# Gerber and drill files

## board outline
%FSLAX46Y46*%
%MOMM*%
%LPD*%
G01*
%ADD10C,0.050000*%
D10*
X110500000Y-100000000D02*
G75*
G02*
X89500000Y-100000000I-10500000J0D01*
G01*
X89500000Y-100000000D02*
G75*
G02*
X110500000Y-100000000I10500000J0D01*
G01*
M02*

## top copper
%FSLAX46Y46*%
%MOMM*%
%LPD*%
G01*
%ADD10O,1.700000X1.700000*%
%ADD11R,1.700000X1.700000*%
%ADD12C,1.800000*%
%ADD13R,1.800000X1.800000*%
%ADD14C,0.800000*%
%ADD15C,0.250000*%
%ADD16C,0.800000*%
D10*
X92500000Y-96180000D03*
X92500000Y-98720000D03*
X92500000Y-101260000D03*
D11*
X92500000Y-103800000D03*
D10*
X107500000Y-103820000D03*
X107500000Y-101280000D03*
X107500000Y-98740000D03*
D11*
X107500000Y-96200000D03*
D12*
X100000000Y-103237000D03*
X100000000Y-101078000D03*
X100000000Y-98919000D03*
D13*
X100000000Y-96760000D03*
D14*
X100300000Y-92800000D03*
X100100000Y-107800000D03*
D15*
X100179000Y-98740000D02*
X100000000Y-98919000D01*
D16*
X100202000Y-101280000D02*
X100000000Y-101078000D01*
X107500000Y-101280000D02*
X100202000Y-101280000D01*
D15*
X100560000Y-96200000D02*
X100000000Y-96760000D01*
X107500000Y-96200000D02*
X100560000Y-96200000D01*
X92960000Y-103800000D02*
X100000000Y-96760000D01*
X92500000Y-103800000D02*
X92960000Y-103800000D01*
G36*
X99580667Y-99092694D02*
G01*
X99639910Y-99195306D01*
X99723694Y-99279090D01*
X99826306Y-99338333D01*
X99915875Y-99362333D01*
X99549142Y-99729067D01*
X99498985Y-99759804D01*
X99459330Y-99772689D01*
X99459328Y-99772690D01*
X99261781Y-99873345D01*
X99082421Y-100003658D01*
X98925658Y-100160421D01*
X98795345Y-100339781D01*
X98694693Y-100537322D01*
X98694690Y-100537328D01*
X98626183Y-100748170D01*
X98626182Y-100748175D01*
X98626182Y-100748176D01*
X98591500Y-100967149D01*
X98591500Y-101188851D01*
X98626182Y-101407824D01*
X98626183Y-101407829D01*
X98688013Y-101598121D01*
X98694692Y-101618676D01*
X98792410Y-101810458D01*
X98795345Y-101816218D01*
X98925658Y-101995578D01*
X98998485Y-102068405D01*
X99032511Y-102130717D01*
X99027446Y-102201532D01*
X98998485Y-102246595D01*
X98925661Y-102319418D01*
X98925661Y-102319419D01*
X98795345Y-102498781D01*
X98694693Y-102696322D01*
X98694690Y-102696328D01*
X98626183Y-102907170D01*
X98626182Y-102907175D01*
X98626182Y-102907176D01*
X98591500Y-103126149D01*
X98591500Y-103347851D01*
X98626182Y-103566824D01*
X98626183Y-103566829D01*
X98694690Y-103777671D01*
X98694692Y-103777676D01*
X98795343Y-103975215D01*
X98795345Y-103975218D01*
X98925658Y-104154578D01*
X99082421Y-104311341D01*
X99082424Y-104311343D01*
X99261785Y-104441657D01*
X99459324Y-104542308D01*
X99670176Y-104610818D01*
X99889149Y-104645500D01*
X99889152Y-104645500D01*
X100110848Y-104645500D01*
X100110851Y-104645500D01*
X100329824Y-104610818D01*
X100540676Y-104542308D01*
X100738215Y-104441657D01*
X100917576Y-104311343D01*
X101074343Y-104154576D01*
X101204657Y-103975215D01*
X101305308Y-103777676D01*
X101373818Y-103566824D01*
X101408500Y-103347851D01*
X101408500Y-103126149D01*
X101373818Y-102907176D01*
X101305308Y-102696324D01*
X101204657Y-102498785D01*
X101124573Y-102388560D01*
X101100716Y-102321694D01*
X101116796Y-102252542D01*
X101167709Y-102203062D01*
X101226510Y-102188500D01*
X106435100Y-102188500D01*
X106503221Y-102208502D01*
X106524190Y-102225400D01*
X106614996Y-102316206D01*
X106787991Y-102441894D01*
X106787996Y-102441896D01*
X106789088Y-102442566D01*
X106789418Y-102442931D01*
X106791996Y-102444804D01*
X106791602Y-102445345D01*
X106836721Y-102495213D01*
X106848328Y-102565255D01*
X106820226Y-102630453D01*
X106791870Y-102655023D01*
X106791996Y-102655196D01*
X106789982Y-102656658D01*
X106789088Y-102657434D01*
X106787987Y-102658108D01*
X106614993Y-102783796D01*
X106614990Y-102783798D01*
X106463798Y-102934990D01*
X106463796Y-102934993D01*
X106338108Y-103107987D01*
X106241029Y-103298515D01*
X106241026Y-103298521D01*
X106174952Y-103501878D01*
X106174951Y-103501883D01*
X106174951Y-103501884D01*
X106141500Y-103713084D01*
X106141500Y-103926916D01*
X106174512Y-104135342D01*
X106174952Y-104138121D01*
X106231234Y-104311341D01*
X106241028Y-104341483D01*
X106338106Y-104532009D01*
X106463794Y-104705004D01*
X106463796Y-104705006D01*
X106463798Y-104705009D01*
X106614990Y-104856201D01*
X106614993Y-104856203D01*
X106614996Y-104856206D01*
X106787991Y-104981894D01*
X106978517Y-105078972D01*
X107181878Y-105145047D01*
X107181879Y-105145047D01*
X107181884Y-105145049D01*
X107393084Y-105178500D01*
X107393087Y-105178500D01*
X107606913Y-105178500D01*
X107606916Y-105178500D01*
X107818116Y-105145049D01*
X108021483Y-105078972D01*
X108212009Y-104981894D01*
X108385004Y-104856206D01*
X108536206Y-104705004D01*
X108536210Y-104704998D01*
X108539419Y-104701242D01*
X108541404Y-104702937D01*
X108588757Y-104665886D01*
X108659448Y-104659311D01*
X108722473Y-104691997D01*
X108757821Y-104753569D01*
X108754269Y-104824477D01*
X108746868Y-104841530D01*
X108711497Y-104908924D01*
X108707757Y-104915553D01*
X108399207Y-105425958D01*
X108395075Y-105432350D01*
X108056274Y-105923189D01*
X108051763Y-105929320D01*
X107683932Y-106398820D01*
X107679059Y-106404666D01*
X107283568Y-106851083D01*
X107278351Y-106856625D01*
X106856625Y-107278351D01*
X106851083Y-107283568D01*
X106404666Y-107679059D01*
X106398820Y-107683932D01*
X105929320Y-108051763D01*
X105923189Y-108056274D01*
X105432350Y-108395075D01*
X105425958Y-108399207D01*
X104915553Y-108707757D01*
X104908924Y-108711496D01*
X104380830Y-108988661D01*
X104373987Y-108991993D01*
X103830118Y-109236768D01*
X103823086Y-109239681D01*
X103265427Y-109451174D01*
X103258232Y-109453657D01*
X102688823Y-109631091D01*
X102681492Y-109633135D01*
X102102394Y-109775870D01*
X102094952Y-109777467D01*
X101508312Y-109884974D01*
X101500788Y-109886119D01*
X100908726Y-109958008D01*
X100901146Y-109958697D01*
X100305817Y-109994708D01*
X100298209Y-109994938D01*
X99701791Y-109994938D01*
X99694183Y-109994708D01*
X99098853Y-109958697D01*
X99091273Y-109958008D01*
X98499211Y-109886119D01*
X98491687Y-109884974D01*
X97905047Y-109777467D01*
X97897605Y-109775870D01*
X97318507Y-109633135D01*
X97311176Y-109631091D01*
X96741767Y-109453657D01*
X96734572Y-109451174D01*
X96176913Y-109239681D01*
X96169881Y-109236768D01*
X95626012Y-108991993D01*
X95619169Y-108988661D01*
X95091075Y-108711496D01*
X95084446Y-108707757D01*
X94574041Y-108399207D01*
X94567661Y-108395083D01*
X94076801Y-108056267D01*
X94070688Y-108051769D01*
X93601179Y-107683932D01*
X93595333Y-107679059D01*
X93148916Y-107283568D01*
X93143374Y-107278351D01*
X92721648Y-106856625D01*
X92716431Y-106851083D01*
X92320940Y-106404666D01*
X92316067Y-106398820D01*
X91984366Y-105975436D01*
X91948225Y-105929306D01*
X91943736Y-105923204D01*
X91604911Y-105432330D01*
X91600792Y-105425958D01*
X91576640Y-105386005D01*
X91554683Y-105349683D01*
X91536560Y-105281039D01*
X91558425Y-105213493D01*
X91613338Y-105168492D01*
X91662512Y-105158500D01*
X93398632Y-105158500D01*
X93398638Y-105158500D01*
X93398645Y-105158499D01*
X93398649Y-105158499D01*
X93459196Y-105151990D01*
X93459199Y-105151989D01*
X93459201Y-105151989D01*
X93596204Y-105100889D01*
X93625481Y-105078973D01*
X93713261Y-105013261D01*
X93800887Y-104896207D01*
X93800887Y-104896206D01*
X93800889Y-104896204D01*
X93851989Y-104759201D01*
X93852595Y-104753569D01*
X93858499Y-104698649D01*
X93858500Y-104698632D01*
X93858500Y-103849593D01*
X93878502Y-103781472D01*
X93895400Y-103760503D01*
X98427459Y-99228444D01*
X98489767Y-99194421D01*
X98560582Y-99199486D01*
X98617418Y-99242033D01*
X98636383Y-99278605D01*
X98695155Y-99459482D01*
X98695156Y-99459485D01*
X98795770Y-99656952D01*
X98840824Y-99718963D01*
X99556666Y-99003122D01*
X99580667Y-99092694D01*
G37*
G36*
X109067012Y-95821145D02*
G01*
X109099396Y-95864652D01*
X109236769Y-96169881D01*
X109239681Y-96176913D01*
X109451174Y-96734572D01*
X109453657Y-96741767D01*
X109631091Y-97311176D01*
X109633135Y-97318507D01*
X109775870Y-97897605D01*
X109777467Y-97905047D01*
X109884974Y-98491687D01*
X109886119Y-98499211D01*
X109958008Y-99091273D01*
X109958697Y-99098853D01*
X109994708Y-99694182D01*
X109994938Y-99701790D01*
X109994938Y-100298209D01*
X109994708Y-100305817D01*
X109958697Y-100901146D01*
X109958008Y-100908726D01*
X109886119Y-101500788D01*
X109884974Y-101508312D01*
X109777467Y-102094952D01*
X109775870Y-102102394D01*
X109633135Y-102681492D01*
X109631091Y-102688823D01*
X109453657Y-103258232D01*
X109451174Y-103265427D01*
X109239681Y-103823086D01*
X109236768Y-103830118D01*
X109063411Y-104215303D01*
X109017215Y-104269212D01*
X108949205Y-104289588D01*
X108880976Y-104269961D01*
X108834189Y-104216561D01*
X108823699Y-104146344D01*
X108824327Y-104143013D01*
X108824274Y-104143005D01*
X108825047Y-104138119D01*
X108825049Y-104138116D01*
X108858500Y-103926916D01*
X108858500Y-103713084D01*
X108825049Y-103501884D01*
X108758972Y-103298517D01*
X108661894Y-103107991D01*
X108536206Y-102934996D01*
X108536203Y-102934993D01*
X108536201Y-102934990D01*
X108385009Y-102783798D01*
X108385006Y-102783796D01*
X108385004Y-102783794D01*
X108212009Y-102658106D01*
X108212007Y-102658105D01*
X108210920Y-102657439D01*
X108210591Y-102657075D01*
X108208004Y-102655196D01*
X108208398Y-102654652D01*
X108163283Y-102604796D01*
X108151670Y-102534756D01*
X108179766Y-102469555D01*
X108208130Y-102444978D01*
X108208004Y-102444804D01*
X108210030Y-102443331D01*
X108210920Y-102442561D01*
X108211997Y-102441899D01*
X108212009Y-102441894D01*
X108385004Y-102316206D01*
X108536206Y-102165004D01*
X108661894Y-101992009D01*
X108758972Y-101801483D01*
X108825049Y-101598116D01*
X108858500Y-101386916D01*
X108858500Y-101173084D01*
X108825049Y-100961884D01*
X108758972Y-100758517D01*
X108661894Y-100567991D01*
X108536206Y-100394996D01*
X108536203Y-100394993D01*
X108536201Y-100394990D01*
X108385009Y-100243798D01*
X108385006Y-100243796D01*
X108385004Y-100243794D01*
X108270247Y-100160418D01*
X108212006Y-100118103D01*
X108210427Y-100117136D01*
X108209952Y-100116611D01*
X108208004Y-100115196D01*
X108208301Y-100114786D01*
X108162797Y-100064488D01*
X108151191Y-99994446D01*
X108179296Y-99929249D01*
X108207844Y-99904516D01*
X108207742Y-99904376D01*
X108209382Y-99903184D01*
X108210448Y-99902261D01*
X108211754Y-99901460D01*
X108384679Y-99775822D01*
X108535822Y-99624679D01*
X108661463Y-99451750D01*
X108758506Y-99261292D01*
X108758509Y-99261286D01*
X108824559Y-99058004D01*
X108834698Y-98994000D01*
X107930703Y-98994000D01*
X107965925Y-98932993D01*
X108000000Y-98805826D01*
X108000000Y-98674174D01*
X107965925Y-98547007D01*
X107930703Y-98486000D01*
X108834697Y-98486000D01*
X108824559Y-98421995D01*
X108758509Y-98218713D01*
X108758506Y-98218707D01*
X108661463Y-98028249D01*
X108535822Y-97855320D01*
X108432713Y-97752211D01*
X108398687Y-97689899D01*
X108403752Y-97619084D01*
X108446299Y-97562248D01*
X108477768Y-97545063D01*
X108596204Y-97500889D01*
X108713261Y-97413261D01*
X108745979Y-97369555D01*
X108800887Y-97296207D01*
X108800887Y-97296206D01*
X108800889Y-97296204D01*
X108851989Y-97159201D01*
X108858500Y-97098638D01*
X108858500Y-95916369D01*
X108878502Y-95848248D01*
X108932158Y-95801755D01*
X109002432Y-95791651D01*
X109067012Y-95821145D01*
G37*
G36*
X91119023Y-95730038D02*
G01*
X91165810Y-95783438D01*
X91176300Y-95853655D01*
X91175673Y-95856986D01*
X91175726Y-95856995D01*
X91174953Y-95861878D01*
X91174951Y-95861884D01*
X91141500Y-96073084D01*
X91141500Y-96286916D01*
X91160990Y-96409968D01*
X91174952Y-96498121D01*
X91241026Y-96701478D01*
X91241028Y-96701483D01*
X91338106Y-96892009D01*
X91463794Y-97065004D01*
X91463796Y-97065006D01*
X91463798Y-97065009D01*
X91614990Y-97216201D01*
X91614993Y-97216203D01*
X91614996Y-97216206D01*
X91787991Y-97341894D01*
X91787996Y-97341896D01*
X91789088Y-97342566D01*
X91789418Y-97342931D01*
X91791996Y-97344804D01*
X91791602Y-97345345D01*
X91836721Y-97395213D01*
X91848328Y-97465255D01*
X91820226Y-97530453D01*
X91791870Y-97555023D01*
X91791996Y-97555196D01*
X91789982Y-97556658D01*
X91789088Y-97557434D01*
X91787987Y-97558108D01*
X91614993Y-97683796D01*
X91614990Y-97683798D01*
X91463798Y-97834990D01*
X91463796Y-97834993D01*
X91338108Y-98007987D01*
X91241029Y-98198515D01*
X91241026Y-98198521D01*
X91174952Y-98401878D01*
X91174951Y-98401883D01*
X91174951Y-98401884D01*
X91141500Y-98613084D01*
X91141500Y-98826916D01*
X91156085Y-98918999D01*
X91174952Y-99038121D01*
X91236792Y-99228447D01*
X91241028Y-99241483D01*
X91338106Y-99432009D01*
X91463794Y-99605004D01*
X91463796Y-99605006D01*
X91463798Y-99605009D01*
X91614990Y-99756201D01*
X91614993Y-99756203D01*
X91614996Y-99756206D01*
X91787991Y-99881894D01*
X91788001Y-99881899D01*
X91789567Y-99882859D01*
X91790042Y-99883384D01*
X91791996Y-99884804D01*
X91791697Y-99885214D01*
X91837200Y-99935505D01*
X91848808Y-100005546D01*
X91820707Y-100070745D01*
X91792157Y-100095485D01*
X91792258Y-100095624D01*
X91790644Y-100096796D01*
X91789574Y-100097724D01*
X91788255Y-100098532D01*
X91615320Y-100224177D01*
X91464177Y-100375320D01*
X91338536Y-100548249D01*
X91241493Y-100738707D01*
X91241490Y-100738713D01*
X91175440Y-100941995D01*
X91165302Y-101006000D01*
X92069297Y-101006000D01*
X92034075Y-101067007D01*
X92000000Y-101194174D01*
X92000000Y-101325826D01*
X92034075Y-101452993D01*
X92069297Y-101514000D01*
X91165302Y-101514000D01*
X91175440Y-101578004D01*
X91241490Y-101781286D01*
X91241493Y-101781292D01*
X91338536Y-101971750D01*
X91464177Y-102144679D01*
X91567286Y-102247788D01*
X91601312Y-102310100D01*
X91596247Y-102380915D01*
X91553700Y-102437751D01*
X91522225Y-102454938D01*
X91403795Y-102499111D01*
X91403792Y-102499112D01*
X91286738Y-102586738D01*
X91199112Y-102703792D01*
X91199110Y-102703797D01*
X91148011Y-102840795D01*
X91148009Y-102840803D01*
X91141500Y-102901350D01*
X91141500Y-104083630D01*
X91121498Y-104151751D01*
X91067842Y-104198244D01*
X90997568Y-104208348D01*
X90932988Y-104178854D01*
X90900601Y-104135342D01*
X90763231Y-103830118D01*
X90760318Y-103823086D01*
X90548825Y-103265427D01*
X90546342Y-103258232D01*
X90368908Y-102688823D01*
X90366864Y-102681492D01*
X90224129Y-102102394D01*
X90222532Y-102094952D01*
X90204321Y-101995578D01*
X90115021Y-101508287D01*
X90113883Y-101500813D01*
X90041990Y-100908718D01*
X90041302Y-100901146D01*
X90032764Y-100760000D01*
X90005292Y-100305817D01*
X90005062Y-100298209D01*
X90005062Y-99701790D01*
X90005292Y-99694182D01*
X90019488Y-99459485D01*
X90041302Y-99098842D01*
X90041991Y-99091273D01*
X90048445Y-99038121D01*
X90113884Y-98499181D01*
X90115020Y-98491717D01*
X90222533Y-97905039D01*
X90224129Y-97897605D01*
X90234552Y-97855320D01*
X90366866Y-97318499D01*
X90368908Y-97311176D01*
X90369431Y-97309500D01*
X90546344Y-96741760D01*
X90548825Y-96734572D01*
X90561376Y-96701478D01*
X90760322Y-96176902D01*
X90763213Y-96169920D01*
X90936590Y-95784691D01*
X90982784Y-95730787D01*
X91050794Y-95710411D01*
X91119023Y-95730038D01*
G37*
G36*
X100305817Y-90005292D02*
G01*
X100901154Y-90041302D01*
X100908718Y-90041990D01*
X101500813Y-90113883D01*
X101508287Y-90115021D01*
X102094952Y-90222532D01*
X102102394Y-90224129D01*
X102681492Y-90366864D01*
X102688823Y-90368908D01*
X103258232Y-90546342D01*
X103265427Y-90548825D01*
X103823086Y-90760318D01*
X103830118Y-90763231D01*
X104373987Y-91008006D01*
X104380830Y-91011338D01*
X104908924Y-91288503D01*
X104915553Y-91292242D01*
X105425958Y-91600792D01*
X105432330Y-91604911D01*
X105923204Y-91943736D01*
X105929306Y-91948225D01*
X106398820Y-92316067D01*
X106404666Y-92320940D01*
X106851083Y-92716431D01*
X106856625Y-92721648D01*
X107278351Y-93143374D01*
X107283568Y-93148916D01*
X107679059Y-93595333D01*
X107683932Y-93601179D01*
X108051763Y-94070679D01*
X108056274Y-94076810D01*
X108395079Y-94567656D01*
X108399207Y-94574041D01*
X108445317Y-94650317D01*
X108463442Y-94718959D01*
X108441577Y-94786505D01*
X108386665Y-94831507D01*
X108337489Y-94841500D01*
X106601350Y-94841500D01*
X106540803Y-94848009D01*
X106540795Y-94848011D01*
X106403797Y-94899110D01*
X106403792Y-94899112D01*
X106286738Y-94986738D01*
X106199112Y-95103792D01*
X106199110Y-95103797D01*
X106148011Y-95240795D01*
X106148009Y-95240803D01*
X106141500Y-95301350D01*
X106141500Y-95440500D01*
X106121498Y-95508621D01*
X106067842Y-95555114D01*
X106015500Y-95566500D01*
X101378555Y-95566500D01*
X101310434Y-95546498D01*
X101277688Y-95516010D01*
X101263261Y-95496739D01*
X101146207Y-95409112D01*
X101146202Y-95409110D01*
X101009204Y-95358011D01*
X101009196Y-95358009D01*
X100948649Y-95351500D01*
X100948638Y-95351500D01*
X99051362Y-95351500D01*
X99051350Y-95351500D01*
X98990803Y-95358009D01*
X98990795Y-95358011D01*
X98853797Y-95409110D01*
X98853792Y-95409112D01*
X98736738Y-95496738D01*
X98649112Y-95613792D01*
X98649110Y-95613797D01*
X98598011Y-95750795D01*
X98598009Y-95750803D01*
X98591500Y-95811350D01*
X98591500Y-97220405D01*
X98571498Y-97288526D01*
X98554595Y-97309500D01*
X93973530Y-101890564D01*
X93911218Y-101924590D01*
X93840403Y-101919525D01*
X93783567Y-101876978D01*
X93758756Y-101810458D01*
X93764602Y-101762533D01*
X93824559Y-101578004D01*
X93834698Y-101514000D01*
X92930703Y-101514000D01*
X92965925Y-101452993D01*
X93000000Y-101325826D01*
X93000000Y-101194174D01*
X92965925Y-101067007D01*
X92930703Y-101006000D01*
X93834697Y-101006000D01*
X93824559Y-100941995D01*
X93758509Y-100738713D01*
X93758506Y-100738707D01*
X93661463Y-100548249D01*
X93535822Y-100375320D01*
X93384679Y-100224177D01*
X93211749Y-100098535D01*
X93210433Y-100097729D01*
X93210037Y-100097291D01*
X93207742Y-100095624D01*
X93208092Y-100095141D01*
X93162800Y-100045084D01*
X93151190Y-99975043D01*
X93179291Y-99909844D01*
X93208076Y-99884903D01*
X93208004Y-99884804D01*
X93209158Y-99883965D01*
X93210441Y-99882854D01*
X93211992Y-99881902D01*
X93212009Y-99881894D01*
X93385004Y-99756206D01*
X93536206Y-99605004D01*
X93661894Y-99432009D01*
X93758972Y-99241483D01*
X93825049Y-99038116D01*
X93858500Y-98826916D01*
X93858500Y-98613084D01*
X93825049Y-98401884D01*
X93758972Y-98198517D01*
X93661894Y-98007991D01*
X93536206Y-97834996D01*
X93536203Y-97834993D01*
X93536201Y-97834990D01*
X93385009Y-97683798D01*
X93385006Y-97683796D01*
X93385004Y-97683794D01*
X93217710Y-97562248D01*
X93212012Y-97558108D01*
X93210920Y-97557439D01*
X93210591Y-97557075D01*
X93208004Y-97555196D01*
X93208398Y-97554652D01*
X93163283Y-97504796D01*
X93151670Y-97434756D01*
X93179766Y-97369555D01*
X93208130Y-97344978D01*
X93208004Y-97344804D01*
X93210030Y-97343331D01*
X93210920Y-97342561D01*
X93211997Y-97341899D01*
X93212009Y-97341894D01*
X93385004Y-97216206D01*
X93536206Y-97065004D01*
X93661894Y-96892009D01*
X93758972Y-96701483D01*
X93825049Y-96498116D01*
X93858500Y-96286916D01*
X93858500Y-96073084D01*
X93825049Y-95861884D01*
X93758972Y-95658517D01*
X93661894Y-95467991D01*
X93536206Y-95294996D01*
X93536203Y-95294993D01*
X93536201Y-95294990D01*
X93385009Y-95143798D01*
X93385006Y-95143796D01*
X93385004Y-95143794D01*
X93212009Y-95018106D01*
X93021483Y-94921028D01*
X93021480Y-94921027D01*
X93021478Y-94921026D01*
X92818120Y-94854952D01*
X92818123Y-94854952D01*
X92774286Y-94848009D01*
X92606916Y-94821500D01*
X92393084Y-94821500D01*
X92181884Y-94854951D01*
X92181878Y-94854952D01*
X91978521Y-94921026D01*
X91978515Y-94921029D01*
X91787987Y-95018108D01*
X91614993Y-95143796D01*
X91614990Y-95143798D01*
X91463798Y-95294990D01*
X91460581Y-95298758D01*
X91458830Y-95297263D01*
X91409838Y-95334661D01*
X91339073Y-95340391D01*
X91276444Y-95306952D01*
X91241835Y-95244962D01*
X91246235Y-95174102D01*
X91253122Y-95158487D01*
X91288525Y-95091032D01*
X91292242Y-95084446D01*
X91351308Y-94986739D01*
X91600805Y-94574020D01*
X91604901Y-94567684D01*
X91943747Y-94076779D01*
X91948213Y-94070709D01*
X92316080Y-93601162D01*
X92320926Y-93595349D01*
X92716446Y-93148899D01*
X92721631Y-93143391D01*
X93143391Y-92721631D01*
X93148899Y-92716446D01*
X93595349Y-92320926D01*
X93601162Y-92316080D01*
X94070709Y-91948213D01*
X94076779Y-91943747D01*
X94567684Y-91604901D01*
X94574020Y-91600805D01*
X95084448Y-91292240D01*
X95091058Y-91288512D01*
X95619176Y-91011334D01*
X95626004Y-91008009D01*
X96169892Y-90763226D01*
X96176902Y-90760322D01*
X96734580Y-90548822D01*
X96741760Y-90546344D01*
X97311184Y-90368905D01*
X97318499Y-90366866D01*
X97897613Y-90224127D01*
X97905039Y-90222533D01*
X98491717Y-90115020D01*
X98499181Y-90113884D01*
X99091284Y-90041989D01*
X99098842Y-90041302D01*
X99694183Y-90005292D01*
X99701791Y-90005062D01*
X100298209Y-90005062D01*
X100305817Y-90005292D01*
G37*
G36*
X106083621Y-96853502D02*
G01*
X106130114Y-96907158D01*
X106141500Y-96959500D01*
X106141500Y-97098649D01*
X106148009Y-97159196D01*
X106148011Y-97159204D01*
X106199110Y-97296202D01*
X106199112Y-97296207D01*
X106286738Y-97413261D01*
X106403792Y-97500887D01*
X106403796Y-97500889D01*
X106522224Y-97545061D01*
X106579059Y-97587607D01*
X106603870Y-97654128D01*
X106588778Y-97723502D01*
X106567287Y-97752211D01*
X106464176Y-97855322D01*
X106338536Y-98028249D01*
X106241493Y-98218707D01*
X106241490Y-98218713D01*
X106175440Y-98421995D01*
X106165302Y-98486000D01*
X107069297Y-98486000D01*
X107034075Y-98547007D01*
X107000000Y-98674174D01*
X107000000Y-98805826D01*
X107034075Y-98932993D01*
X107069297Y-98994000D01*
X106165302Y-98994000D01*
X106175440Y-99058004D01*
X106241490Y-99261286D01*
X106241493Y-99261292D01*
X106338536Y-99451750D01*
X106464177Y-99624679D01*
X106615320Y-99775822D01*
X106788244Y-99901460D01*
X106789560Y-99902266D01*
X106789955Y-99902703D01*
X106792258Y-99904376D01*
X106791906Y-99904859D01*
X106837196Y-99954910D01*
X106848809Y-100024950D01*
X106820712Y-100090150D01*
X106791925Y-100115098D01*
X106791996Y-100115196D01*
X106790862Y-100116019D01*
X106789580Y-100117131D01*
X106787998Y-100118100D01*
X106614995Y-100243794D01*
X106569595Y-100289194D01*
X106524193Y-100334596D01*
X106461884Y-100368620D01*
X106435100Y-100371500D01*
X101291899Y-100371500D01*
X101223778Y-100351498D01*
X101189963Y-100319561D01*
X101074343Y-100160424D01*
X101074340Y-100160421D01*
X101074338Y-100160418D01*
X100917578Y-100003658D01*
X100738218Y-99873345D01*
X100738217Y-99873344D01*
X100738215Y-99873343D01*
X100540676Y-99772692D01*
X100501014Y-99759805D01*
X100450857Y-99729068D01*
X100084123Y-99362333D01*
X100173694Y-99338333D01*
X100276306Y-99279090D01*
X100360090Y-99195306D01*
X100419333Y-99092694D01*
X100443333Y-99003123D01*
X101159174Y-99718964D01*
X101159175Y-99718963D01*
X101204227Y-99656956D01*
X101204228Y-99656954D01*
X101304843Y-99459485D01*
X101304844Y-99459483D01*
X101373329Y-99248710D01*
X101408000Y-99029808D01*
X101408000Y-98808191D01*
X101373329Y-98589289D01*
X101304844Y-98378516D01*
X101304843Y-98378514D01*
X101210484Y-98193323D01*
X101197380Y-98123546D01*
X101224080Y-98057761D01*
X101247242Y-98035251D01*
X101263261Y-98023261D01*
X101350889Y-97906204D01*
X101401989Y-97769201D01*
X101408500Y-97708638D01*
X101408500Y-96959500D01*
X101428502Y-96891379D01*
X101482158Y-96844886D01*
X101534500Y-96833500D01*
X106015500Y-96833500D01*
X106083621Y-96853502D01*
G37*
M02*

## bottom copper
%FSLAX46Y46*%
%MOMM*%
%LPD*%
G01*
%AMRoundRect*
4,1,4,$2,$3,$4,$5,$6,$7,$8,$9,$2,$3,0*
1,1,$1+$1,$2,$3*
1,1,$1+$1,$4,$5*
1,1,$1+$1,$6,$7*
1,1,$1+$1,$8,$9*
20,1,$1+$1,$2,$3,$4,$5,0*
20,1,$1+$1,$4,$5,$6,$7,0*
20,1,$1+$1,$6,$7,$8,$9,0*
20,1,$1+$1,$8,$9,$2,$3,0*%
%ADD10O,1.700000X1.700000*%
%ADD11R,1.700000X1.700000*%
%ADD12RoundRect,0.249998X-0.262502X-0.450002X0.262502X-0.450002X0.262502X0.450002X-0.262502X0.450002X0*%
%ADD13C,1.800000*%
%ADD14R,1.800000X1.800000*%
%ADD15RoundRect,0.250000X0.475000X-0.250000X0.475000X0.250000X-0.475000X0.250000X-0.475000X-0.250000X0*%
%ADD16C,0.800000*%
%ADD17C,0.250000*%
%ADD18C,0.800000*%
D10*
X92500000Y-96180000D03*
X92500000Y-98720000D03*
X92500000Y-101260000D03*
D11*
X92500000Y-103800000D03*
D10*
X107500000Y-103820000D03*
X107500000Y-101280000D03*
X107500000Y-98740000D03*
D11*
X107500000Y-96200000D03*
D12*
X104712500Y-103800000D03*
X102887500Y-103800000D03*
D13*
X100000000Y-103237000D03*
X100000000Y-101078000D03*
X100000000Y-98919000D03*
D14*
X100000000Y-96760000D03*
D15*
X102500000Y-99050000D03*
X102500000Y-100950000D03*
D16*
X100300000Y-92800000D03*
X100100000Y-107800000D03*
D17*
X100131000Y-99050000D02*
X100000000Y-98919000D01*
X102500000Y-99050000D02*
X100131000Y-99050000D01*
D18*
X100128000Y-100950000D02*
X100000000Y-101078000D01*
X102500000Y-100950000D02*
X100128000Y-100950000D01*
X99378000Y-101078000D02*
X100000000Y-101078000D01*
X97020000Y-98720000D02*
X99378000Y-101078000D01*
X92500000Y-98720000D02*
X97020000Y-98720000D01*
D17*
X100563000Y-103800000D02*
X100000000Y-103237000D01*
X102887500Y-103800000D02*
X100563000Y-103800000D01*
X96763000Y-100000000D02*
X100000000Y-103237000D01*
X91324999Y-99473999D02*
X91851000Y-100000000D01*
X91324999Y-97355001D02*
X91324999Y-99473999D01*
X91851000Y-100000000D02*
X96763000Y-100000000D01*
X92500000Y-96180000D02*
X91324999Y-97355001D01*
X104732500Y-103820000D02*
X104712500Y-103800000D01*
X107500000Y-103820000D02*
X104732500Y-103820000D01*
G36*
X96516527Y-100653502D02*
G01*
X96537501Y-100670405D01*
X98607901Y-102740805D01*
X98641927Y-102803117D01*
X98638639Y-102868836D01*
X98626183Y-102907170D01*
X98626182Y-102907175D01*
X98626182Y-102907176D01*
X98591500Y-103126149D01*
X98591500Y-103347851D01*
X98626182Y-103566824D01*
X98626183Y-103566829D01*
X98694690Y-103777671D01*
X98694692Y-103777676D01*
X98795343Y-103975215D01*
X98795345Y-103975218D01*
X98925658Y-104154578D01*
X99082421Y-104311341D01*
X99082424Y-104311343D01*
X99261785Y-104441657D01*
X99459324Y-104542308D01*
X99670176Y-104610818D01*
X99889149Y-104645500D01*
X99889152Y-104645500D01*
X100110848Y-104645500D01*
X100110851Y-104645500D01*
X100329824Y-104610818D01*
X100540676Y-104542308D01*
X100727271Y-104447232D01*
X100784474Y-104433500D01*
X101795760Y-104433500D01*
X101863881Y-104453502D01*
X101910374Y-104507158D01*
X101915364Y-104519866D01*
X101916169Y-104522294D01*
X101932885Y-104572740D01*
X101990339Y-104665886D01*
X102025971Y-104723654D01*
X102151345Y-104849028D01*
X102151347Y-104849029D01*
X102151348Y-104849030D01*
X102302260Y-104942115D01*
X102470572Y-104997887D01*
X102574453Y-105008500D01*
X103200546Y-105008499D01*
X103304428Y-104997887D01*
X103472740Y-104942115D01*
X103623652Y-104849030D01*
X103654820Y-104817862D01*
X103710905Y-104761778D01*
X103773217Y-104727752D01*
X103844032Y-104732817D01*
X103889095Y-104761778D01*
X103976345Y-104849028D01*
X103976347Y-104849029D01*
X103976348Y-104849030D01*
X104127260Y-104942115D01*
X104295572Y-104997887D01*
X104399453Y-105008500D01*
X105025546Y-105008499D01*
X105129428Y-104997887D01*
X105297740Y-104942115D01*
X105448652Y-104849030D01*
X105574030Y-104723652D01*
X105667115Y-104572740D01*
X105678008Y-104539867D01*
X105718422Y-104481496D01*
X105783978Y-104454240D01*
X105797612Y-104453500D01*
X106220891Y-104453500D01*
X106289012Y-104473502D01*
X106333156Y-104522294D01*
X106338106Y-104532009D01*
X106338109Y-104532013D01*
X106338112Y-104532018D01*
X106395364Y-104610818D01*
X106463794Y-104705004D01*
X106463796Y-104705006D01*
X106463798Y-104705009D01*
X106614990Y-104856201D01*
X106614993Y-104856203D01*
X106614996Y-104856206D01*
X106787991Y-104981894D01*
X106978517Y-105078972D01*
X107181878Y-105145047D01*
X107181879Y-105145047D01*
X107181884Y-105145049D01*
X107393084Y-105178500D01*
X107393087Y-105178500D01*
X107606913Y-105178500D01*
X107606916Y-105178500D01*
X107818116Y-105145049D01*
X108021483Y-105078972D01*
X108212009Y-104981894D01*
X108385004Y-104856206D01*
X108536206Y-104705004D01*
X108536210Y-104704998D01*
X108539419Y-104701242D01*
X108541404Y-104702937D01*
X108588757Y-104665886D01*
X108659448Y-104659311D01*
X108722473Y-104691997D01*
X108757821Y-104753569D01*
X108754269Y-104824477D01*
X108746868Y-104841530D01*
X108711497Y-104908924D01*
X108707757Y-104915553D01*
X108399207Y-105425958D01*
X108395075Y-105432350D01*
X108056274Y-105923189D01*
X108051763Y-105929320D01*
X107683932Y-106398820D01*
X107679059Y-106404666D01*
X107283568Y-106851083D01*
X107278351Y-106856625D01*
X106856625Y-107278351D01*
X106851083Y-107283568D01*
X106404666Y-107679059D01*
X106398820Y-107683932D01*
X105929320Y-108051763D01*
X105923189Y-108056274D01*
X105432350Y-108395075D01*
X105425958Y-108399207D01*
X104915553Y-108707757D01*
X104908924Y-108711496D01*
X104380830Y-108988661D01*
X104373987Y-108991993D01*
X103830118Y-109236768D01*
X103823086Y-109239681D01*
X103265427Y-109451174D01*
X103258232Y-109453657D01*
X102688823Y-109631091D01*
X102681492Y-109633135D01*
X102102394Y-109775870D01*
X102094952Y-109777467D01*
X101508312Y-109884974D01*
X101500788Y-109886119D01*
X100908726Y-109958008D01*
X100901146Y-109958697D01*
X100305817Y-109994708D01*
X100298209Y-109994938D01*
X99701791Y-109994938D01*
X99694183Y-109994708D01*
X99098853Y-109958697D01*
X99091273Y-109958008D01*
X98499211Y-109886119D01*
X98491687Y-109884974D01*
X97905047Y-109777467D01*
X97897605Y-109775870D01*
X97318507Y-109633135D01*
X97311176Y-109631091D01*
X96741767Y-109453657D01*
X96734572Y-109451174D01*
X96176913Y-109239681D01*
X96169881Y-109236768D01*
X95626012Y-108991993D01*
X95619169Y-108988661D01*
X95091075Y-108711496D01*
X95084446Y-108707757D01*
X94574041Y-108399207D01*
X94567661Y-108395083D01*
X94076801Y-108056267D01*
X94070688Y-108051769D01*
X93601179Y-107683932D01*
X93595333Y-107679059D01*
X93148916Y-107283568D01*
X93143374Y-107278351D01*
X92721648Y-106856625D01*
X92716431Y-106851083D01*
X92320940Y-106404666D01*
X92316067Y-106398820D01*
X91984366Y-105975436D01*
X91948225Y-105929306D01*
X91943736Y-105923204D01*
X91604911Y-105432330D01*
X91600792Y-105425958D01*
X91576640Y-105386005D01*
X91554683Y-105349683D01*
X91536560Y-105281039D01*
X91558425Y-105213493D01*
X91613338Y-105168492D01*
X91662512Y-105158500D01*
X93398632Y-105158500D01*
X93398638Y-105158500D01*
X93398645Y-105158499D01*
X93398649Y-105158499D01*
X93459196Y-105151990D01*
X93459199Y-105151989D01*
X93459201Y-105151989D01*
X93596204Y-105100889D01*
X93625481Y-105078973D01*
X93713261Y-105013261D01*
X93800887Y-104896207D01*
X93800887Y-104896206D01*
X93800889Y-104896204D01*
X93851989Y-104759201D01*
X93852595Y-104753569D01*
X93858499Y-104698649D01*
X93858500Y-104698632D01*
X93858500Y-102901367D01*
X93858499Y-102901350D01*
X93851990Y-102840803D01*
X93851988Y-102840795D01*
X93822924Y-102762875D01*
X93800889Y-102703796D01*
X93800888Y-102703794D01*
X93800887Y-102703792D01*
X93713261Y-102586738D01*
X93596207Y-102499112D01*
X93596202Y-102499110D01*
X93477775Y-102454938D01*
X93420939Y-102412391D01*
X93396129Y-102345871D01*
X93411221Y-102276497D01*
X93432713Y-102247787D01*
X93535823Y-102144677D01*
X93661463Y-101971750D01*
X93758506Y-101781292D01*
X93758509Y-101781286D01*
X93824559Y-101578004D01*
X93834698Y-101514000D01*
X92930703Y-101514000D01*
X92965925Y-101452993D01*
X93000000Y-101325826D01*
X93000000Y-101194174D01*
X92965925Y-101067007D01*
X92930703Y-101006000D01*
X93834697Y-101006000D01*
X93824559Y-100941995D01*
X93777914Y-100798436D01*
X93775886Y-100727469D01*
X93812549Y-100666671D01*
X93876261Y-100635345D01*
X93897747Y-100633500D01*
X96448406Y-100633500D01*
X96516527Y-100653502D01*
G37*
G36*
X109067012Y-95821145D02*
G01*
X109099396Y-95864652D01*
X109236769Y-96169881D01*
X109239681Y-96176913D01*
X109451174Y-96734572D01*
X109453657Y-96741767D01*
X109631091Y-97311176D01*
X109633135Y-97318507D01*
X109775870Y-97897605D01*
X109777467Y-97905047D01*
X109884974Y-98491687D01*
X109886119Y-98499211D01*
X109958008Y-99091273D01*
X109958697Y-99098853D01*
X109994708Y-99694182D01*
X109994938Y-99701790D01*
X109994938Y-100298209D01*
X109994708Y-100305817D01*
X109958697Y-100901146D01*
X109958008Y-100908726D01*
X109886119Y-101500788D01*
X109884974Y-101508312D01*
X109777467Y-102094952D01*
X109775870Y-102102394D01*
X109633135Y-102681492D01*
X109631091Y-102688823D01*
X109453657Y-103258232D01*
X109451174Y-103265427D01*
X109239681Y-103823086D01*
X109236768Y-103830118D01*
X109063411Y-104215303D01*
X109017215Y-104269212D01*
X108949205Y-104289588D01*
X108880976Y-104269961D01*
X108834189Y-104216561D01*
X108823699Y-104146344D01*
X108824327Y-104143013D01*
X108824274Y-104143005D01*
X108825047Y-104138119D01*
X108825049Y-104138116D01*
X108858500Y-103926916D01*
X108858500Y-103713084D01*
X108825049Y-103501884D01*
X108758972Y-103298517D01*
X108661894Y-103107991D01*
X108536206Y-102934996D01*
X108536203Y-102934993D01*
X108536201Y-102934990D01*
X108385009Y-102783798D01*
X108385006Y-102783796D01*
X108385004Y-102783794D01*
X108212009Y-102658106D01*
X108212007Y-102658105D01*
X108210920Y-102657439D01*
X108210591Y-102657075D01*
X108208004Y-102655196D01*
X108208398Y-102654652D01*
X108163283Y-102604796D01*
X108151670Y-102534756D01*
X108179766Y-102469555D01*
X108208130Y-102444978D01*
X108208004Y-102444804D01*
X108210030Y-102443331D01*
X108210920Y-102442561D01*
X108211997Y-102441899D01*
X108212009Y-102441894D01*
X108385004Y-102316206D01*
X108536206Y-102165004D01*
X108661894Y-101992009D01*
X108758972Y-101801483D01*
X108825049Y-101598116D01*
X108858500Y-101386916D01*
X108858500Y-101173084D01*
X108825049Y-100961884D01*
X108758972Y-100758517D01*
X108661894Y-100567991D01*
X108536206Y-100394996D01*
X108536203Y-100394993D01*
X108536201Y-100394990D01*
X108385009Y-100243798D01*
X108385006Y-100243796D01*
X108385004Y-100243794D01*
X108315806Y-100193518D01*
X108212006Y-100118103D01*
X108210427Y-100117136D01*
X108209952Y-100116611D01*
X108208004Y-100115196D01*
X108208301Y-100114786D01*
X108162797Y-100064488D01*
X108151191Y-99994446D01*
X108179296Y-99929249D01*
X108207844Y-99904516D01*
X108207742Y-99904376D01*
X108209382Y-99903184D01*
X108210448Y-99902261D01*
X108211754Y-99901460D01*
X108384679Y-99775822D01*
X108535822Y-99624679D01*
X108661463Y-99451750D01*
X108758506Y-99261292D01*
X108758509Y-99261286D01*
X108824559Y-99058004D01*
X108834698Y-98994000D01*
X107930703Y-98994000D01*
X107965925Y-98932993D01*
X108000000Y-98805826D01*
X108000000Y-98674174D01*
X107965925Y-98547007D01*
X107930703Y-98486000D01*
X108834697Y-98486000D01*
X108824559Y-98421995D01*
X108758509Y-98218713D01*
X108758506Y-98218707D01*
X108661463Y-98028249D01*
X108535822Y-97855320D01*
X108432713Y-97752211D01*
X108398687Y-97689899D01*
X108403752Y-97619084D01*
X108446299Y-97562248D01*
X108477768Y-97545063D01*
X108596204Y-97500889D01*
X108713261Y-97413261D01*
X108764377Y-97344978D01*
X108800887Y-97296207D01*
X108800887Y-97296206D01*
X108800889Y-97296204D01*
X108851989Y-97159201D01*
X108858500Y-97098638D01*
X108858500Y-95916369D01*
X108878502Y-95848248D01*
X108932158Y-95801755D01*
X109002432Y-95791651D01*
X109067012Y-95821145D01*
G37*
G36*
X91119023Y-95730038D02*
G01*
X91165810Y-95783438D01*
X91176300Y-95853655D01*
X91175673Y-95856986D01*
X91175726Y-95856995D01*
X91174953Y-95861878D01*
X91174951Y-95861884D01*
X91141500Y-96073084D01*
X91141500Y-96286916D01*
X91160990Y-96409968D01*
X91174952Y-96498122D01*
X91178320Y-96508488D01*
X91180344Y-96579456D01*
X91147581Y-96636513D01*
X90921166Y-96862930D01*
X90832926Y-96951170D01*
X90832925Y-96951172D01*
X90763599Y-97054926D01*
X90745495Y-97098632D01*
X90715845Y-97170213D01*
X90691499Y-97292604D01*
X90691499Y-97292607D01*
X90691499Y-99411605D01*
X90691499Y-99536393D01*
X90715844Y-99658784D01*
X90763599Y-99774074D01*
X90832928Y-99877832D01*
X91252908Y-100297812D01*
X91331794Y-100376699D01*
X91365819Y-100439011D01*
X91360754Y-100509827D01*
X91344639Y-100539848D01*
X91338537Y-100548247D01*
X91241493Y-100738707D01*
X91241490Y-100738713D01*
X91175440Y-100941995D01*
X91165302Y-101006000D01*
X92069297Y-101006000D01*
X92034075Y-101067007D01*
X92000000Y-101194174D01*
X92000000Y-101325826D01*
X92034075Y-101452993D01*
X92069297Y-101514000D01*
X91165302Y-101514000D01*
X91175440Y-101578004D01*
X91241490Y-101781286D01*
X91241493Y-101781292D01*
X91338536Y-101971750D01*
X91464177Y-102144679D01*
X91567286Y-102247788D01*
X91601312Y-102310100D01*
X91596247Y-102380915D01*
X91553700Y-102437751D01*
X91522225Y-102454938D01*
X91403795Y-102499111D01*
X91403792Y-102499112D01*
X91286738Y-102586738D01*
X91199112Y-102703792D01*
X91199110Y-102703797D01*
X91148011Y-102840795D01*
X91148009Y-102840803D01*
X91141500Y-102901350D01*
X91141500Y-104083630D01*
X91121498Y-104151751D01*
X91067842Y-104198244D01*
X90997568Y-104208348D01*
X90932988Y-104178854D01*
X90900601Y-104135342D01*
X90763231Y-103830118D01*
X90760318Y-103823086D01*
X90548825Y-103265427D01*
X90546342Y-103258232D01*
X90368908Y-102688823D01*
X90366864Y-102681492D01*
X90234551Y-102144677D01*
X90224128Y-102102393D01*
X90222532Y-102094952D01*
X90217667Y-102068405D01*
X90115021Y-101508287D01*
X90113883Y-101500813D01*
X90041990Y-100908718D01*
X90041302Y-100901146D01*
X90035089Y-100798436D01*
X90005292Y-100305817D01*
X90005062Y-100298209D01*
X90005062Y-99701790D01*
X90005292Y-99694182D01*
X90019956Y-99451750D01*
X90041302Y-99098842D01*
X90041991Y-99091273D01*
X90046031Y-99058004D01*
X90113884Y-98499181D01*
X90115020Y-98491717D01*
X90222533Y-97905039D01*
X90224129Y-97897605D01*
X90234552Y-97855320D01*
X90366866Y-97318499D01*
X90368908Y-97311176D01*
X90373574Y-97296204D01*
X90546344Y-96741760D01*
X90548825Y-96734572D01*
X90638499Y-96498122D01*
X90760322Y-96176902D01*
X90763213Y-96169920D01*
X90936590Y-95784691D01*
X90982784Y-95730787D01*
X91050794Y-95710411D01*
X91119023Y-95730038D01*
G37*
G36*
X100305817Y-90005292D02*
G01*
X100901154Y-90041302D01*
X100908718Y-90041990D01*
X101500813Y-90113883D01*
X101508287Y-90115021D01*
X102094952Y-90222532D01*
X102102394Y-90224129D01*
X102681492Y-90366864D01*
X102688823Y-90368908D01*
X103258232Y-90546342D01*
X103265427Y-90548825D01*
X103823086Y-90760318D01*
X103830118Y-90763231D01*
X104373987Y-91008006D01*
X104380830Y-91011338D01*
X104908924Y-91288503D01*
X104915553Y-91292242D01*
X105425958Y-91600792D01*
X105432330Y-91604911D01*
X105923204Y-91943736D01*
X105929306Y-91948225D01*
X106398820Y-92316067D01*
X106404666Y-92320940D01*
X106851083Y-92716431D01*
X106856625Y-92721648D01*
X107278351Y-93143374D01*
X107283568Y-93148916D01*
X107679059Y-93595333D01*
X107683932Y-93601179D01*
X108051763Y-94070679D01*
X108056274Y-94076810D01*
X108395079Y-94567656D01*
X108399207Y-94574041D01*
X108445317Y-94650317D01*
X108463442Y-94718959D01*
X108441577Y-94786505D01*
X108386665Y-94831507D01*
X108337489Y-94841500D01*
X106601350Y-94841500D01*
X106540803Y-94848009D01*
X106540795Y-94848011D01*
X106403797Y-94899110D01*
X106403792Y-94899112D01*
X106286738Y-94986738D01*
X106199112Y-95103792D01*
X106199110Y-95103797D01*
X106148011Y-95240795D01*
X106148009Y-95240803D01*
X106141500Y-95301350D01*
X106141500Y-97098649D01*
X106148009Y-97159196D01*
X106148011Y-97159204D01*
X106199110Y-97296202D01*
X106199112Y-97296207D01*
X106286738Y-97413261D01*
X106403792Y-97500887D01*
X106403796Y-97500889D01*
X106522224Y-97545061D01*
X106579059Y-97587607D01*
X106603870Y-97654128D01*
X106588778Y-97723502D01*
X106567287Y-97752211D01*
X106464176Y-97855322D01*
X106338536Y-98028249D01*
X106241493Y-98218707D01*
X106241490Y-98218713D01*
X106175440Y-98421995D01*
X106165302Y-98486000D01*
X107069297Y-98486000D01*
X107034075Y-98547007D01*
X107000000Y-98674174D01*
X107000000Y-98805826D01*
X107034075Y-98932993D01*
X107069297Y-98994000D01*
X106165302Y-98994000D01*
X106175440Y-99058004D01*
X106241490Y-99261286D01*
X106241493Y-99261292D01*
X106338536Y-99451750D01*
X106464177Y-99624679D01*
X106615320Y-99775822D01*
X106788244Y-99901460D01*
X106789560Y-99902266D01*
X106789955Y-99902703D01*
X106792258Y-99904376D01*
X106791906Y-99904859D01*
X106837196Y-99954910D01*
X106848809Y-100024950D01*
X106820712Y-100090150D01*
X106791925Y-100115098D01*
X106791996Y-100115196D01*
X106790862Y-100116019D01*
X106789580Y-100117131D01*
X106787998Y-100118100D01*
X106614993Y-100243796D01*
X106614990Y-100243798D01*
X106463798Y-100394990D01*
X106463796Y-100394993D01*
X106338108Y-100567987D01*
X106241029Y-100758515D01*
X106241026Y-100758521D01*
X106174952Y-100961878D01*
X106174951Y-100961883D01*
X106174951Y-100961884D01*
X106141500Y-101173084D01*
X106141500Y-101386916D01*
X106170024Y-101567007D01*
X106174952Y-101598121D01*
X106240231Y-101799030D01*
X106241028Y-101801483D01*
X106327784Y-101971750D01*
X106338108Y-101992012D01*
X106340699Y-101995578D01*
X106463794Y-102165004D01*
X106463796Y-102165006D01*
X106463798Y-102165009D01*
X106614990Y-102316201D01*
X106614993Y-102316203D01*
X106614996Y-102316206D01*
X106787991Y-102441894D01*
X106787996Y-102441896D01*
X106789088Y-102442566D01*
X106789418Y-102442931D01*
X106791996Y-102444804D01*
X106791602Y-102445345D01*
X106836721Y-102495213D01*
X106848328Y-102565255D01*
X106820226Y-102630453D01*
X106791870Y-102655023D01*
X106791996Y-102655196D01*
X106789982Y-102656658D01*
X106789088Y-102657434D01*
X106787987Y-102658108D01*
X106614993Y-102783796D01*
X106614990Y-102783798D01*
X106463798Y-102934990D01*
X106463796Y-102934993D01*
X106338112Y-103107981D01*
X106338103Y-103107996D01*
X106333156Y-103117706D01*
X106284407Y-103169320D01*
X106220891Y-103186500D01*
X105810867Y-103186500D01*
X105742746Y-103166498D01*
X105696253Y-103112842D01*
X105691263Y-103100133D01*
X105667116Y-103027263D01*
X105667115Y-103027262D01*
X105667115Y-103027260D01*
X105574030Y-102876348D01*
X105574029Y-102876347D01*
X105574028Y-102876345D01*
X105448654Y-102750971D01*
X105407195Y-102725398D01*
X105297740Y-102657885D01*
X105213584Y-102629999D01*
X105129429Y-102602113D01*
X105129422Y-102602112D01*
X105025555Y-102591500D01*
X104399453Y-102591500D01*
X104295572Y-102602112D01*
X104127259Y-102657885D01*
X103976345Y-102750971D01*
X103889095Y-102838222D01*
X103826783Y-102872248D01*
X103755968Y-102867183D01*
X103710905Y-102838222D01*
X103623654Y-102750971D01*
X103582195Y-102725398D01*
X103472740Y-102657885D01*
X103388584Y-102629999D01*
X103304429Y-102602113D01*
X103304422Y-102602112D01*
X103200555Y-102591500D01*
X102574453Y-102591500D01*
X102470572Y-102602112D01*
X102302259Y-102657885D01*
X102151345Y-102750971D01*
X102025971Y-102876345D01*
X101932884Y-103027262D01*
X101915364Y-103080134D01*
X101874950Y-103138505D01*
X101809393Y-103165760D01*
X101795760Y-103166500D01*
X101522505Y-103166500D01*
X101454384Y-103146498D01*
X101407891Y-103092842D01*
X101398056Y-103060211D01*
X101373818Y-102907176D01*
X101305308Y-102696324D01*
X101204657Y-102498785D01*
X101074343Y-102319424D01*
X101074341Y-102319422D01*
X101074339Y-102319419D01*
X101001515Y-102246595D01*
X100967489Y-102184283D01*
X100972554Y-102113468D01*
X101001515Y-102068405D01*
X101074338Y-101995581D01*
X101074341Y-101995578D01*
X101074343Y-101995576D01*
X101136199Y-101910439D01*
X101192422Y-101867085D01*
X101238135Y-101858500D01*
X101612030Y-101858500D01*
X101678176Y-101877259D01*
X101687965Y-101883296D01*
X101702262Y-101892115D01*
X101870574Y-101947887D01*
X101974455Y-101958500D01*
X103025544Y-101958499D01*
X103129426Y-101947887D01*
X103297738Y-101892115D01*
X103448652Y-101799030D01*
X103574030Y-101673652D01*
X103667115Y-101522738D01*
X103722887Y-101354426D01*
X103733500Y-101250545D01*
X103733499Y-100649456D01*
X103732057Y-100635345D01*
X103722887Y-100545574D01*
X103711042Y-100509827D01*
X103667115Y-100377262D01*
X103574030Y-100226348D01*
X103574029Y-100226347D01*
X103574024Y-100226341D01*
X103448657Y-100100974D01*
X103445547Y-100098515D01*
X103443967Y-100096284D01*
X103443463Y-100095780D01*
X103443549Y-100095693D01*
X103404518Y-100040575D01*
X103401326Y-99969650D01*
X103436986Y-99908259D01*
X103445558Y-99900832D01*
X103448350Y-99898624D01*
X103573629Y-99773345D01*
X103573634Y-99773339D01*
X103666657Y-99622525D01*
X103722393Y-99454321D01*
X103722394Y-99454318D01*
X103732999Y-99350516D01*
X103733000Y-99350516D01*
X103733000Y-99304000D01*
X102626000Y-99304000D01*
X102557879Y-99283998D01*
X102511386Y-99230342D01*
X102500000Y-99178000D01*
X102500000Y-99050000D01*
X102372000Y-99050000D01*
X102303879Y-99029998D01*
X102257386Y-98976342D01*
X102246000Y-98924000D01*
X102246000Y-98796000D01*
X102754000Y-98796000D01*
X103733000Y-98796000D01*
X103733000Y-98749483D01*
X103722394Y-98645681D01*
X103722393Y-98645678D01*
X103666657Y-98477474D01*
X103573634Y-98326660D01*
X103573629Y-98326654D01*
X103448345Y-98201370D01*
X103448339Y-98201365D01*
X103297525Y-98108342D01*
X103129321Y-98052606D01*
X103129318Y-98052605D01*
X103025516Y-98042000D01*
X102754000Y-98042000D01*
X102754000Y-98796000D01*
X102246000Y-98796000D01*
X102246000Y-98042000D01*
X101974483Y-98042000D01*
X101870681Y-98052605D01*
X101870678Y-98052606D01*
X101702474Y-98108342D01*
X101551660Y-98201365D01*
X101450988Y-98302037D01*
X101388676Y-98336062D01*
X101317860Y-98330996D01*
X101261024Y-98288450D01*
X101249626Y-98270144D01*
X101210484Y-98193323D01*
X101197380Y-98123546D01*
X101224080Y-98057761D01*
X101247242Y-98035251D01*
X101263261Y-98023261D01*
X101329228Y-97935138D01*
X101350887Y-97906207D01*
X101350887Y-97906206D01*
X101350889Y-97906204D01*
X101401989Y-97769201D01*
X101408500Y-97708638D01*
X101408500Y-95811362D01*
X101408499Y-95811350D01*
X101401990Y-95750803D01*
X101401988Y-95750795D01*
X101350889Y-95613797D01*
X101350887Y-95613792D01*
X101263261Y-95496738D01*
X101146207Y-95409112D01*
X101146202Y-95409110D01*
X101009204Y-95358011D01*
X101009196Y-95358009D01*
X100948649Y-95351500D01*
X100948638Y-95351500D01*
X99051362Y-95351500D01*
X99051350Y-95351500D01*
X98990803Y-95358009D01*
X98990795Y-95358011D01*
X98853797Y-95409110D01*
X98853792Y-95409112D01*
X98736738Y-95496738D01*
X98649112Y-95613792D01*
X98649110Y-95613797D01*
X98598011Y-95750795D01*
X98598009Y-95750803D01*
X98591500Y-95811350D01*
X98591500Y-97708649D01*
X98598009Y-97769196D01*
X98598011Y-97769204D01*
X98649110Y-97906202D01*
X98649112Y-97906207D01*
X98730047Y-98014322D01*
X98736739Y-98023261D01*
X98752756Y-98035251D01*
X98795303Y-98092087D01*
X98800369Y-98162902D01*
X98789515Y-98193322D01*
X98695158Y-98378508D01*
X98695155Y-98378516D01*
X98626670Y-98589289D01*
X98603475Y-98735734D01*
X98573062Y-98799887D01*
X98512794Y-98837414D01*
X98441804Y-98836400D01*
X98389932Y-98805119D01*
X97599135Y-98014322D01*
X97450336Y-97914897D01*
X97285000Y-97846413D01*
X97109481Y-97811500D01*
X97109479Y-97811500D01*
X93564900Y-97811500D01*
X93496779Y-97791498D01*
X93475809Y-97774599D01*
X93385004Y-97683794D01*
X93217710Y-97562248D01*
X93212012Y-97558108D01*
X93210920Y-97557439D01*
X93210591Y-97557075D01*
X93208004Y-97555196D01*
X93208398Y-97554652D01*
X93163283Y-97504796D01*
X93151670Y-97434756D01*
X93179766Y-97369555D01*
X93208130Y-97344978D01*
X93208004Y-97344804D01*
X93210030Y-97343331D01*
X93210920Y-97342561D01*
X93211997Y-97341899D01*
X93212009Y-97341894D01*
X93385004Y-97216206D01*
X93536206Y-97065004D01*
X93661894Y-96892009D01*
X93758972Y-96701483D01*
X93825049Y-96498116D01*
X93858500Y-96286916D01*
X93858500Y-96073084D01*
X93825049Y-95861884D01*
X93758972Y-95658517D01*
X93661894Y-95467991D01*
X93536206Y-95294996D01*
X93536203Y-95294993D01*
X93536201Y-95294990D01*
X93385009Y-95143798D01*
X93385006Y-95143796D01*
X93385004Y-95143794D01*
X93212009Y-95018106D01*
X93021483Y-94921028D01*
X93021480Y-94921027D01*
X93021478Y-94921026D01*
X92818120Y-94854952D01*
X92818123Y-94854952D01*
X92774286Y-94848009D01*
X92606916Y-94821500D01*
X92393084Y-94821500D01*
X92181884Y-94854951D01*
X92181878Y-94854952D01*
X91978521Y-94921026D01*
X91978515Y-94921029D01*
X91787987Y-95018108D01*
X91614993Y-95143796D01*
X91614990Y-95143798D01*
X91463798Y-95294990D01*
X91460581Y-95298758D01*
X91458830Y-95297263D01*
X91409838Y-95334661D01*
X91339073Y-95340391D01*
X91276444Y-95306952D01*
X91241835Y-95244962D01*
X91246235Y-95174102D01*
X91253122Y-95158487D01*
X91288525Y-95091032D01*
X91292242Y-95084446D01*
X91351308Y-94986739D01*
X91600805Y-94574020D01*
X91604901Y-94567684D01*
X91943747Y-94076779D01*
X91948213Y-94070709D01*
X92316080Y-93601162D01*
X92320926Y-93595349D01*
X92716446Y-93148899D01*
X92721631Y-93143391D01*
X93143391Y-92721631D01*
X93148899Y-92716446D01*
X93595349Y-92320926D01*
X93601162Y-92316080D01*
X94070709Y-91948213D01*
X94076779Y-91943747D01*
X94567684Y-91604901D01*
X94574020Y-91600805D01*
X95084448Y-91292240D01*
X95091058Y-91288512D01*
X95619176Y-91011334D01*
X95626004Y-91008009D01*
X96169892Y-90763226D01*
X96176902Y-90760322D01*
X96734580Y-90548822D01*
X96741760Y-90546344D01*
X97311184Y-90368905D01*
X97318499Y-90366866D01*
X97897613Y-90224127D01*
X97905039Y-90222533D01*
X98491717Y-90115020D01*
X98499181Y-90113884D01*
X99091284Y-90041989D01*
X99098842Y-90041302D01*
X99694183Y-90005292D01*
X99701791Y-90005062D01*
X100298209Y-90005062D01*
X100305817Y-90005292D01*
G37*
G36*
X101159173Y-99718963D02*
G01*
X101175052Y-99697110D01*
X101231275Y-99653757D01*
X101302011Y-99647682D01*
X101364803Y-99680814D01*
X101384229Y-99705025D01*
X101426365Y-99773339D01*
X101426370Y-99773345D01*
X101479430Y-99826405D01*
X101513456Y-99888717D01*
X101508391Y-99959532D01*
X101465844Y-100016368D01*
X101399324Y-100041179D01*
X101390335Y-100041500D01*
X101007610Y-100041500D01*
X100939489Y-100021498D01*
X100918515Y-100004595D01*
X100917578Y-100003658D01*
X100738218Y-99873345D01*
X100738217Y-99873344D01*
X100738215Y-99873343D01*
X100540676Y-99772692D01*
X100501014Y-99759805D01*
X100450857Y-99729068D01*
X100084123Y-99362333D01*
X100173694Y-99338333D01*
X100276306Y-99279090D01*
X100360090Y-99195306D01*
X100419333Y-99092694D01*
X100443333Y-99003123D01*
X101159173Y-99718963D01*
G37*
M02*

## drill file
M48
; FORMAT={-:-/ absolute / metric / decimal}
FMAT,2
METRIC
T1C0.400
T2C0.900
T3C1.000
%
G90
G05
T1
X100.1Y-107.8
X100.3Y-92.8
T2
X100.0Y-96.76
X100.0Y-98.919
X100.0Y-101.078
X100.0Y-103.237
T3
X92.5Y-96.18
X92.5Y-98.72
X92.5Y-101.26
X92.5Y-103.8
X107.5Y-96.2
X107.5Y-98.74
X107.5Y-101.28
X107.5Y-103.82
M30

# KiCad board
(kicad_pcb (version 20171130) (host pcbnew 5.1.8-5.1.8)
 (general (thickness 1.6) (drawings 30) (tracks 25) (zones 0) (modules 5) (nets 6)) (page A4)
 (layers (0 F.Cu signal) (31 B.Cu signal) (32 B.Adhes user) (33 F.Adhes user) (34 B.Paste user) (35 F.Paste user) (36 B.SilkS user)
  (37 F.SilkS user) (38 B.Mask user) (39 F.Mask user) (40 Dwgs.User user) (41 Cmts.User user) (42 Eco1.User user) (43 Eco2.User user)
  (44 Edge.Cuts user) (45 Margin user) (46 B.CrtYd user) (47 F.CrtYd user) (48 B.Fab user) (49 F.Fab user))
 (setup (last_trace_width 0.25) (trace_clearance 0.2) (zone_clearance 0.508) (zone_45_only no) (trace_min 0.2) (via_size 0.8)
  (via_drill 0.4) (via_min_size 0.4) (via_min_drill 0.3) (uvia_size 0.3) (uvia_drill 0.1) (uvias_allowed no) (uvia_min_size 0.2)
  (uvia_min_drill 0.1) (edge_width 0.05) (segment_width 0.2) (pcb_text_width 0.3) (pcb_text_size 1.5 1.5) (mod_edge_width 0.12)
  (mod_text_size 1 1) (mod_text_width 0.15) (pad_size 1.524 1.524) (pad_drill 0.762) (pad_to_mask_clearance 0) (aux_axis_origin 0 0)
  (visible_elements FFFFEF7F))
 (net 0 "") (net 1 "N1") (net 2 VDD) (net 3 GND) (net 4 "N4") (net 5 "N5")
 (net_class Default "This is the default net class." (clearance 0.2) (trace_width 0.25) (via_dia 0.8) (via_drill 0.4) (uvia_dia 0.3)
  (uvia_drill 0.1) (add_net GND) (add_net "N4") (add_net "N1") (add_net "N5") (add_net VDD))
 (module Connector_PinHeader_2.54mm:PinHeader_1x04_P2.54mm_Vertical (layer B.Cu) (at 92.5 103.8)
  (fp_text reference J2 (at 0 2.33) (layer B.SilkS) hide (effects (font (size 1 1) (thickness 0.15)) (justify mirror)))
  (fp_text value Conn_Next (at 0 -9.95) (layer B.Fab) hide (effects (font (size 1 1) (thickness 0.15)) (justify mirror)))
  (pad 4 thru_hole oval (at 0 -7.62) (size 1.7 1.7) (drill 1) (layers *.Cu *.Mask) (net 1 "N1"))
  (pad 3 thru_hole oval (at 0 -5.08) (size 1.7 1.7) (drill 1) (layers *.Cu *.Mask) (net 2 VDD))
  (pad 2 thru_hole oval (at 0 -2.54) (size 1.7 1.7) (drill 1) (layers *.Cu *.Mask) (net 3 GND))
  (pad 1 thru_hole rect (at 0 0) (size 1.7 1.7) (drill 1) (layers *.Cu *.Mask) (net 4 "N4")))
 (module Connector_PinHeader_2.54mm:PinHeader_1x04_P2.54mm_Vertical (layer B.Cu) (at 107.5 96.2 180)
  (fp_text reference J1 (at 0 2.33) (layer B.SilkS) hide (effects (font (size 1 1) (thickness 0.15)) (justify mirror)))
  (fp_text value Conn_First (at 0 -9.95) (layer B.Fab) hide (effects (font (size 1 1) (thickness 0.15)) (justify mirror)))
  (pad 4 thru_hole oval (at 0 -7.62 180) (size 1.7 1.7) (drill 1) (layers *.Cu *.Mask) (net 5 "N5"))
  (pad 3 thru_hole oval (at 0 -5.08 180) (size 1.7 1.7) (drill 1) (layers *.Cu *.Mask) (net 2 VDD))
  (pad 2 thru_hole oval (at 0 -2.54 180) (size 1.7 1.7) (drill 1) (layers *.Cu *.Mask) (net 3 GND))
  (pad 1 thru_hole rect (at 0 0 180) (size 1.7 1.7) (drill 1) (layers *.Cu *.Mask) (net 4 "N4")))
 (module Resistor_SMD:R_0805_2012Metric (layer B.Cu) (at 103.8 103.8)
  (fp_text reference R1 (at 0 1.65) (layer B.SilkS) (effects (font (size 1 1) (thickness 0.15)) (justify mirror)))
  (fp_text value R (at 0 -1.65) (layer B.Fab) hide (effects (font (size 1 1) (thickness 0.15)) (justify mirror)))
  (pad 2 smd roundrect (at 0.9125 0) (size 1.025 1.4) (layers B.Cu B.Paste B.Mask) (roundrect_rratio 0.2439004878048781) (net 5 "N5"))
  (pad 1 smd roundrect (at -0.9125 0) (size 1.025 1.4) (layers B.Cu B.Paste B.Mask) (roundrect_rratio 0.2439004878048781) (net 1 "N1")))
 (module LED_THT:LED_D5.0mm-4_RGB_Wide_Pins (layer F.Cu) (at 100 96.76 270)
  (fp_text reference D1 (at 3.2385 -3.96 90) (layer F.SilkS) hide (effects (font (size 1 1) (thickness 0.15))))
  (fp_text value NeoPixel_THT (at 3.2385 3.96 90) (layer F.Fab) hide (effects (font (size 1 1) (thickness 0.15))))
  (pad 4 thru_hole circle (at 6.477 0 270) (size 1.8 1.8) (drill 0.9) (layers *.Cu *.Mask) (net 1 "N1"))
  (pad 3 thru_hole circle (at 4.318 0 270) (size 1.8 1.8) (drill 0.9) (layers *.Cu *.Mask) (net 2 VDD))
  (pad 2 thru_hole circle (at 2.159 0 270) (size 1.8 1.8) (drill 0.9) (layers *.Cu *.Mask) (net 3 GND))
  (pad 1 thru_hole rect (at 0 0 270) (size 1.8 1.8) (drill 0.9) (layers *.Cu *.Mask) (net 4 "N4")))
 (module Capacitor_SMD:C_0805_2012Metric (layer B.Cu) (at 102.5 100 90)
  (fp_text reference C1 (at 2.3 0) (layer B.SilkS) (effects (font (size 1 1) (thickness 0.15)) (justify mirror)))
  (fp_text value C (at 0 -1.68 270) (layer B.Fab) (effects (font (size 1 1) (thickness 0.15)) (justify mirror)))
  (pad 2 smd roundrect (at 0.95 0 90) (size 1 1.45) (layers B.Cu B.Paste B.Mask) (roundrect_rratio 0.25) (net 3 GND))
  (pad 1 smd roundrect (at -0.95 0 90) (size 1 1.45) (layers B.Cu B.Paste B.Mask) (roundrect_rratio 0.25) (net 2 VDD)))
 (gr_circle (center 100 100) (end 110.5 100) (layer Edge.Cuts) (width 0.05))
 (segment (start 100.179 98.74) (end 100 98.919) (width 0.25) (layer F.Cu) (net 3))
 (segment (start 100.131 99.05) (end 100 98.919) (width 0.25) (layer B.Cu) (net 3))
 (segment (start 102.5 99.05) (end 100.131 99.05) (width 0.25) (layer B.Cu) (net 3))
 (via (at 100.3 92.8) (size 0.8) (drill 0.4) (layers F.Cu B.Cu) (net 3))
 (via (at 100.1 107.8) (size 0.8) (drill 0.4) (layers F.Cu B.Cu) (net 3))
 (segment (start 100.202 101.28) (end 100 101.078) (width 0.8) (layer F.Cu) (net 2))
 (segment (start 107.5 101.28) (end 100.202 101.28) (width 0.8) (layer F.Cu) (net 2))
 (segment (start 100.128 100.95) (end 100 101.078) (width 0.8) (layer B.Cu) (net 2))
 (segment (start 102.5 100.95) (end 100.128 100.95) (width 0.8) (layer B.Cu) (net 2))
 (segment (start 99.378 101.078) (end 100 101.078) (width 0.8) (layer B.Cu) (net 2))
 (segment (start 97.02 98.72) (end 99.378 101.078) (width 0.8) (layer B.Cu) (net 2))
 (segment (start 92.5 98.72) (end 97.02 98.72) (width 0.8) (layer B.Cu) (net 2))
 (segment (start 100.563 103.8) (end 100 103.237) (width 0.25) (layer B.Cu) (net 1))
 (segment (start 102.8875 103.8) (end 100.563 103.8) (width 0.25) (layer B.Cu) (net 1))
 (segment (start 96.763 100) (end 100 103.237) (width 0.25) (layer B.Cu) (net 1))
 (segment (start 91.324999 99.473999) (end 91.851 100) (width 0.25) (layer B.Cu) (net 1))
 (segment (start 91.324999 97.355001) (end 91.324999 99.473999) (width 0.25) (layer B.Cu) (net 1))
 (segment (start 91.851 100) (end 96.763 100) (width 0.25) (layer B.Cu) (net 1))
 (segment (start 92.5 96.18) (end 91.324999 97.355001) (width 0.25) (layer B.Cu) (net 1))
 (segment (start 100.56 96.2) (end 100 96.76) (width 0.25) (layer F.Cu) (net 4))
 (segment (start 107.5 96.2) (end 100.56 96.2) (width 0.25) (layer F.Cu) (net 4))
 (segment (start 92.96 103.8) (end 100 96.76) (width 0.25) (layer F.Cu) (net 4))
 (segment (start 92.5 103.8) (end 92.96 103.8) (width 0.25) (layer F.Cu) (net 4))
 (segment (start 104.7325 103.82) (end 104.7125 103.8) (width 0.25) (layer B.Cu) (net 5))
 (segment (start 107.5 103.82) (end 104.7325 103.82) (width 0.25) (layer B.Cu) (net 5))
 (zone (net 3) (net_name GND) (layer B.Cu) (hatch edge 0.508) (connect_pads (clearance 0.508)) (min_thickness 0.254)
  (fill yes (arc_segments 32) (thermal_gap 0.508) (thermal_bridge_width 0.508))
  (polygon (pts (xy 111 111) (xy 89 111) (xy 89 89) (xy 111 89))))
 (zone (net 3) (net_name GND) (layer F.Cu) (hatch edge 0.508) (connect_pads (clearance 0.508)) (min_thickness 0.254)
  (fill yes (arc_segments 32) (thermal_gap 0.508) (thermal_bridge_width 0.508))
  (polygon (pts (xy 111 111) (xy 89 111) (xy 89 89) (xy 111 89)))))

